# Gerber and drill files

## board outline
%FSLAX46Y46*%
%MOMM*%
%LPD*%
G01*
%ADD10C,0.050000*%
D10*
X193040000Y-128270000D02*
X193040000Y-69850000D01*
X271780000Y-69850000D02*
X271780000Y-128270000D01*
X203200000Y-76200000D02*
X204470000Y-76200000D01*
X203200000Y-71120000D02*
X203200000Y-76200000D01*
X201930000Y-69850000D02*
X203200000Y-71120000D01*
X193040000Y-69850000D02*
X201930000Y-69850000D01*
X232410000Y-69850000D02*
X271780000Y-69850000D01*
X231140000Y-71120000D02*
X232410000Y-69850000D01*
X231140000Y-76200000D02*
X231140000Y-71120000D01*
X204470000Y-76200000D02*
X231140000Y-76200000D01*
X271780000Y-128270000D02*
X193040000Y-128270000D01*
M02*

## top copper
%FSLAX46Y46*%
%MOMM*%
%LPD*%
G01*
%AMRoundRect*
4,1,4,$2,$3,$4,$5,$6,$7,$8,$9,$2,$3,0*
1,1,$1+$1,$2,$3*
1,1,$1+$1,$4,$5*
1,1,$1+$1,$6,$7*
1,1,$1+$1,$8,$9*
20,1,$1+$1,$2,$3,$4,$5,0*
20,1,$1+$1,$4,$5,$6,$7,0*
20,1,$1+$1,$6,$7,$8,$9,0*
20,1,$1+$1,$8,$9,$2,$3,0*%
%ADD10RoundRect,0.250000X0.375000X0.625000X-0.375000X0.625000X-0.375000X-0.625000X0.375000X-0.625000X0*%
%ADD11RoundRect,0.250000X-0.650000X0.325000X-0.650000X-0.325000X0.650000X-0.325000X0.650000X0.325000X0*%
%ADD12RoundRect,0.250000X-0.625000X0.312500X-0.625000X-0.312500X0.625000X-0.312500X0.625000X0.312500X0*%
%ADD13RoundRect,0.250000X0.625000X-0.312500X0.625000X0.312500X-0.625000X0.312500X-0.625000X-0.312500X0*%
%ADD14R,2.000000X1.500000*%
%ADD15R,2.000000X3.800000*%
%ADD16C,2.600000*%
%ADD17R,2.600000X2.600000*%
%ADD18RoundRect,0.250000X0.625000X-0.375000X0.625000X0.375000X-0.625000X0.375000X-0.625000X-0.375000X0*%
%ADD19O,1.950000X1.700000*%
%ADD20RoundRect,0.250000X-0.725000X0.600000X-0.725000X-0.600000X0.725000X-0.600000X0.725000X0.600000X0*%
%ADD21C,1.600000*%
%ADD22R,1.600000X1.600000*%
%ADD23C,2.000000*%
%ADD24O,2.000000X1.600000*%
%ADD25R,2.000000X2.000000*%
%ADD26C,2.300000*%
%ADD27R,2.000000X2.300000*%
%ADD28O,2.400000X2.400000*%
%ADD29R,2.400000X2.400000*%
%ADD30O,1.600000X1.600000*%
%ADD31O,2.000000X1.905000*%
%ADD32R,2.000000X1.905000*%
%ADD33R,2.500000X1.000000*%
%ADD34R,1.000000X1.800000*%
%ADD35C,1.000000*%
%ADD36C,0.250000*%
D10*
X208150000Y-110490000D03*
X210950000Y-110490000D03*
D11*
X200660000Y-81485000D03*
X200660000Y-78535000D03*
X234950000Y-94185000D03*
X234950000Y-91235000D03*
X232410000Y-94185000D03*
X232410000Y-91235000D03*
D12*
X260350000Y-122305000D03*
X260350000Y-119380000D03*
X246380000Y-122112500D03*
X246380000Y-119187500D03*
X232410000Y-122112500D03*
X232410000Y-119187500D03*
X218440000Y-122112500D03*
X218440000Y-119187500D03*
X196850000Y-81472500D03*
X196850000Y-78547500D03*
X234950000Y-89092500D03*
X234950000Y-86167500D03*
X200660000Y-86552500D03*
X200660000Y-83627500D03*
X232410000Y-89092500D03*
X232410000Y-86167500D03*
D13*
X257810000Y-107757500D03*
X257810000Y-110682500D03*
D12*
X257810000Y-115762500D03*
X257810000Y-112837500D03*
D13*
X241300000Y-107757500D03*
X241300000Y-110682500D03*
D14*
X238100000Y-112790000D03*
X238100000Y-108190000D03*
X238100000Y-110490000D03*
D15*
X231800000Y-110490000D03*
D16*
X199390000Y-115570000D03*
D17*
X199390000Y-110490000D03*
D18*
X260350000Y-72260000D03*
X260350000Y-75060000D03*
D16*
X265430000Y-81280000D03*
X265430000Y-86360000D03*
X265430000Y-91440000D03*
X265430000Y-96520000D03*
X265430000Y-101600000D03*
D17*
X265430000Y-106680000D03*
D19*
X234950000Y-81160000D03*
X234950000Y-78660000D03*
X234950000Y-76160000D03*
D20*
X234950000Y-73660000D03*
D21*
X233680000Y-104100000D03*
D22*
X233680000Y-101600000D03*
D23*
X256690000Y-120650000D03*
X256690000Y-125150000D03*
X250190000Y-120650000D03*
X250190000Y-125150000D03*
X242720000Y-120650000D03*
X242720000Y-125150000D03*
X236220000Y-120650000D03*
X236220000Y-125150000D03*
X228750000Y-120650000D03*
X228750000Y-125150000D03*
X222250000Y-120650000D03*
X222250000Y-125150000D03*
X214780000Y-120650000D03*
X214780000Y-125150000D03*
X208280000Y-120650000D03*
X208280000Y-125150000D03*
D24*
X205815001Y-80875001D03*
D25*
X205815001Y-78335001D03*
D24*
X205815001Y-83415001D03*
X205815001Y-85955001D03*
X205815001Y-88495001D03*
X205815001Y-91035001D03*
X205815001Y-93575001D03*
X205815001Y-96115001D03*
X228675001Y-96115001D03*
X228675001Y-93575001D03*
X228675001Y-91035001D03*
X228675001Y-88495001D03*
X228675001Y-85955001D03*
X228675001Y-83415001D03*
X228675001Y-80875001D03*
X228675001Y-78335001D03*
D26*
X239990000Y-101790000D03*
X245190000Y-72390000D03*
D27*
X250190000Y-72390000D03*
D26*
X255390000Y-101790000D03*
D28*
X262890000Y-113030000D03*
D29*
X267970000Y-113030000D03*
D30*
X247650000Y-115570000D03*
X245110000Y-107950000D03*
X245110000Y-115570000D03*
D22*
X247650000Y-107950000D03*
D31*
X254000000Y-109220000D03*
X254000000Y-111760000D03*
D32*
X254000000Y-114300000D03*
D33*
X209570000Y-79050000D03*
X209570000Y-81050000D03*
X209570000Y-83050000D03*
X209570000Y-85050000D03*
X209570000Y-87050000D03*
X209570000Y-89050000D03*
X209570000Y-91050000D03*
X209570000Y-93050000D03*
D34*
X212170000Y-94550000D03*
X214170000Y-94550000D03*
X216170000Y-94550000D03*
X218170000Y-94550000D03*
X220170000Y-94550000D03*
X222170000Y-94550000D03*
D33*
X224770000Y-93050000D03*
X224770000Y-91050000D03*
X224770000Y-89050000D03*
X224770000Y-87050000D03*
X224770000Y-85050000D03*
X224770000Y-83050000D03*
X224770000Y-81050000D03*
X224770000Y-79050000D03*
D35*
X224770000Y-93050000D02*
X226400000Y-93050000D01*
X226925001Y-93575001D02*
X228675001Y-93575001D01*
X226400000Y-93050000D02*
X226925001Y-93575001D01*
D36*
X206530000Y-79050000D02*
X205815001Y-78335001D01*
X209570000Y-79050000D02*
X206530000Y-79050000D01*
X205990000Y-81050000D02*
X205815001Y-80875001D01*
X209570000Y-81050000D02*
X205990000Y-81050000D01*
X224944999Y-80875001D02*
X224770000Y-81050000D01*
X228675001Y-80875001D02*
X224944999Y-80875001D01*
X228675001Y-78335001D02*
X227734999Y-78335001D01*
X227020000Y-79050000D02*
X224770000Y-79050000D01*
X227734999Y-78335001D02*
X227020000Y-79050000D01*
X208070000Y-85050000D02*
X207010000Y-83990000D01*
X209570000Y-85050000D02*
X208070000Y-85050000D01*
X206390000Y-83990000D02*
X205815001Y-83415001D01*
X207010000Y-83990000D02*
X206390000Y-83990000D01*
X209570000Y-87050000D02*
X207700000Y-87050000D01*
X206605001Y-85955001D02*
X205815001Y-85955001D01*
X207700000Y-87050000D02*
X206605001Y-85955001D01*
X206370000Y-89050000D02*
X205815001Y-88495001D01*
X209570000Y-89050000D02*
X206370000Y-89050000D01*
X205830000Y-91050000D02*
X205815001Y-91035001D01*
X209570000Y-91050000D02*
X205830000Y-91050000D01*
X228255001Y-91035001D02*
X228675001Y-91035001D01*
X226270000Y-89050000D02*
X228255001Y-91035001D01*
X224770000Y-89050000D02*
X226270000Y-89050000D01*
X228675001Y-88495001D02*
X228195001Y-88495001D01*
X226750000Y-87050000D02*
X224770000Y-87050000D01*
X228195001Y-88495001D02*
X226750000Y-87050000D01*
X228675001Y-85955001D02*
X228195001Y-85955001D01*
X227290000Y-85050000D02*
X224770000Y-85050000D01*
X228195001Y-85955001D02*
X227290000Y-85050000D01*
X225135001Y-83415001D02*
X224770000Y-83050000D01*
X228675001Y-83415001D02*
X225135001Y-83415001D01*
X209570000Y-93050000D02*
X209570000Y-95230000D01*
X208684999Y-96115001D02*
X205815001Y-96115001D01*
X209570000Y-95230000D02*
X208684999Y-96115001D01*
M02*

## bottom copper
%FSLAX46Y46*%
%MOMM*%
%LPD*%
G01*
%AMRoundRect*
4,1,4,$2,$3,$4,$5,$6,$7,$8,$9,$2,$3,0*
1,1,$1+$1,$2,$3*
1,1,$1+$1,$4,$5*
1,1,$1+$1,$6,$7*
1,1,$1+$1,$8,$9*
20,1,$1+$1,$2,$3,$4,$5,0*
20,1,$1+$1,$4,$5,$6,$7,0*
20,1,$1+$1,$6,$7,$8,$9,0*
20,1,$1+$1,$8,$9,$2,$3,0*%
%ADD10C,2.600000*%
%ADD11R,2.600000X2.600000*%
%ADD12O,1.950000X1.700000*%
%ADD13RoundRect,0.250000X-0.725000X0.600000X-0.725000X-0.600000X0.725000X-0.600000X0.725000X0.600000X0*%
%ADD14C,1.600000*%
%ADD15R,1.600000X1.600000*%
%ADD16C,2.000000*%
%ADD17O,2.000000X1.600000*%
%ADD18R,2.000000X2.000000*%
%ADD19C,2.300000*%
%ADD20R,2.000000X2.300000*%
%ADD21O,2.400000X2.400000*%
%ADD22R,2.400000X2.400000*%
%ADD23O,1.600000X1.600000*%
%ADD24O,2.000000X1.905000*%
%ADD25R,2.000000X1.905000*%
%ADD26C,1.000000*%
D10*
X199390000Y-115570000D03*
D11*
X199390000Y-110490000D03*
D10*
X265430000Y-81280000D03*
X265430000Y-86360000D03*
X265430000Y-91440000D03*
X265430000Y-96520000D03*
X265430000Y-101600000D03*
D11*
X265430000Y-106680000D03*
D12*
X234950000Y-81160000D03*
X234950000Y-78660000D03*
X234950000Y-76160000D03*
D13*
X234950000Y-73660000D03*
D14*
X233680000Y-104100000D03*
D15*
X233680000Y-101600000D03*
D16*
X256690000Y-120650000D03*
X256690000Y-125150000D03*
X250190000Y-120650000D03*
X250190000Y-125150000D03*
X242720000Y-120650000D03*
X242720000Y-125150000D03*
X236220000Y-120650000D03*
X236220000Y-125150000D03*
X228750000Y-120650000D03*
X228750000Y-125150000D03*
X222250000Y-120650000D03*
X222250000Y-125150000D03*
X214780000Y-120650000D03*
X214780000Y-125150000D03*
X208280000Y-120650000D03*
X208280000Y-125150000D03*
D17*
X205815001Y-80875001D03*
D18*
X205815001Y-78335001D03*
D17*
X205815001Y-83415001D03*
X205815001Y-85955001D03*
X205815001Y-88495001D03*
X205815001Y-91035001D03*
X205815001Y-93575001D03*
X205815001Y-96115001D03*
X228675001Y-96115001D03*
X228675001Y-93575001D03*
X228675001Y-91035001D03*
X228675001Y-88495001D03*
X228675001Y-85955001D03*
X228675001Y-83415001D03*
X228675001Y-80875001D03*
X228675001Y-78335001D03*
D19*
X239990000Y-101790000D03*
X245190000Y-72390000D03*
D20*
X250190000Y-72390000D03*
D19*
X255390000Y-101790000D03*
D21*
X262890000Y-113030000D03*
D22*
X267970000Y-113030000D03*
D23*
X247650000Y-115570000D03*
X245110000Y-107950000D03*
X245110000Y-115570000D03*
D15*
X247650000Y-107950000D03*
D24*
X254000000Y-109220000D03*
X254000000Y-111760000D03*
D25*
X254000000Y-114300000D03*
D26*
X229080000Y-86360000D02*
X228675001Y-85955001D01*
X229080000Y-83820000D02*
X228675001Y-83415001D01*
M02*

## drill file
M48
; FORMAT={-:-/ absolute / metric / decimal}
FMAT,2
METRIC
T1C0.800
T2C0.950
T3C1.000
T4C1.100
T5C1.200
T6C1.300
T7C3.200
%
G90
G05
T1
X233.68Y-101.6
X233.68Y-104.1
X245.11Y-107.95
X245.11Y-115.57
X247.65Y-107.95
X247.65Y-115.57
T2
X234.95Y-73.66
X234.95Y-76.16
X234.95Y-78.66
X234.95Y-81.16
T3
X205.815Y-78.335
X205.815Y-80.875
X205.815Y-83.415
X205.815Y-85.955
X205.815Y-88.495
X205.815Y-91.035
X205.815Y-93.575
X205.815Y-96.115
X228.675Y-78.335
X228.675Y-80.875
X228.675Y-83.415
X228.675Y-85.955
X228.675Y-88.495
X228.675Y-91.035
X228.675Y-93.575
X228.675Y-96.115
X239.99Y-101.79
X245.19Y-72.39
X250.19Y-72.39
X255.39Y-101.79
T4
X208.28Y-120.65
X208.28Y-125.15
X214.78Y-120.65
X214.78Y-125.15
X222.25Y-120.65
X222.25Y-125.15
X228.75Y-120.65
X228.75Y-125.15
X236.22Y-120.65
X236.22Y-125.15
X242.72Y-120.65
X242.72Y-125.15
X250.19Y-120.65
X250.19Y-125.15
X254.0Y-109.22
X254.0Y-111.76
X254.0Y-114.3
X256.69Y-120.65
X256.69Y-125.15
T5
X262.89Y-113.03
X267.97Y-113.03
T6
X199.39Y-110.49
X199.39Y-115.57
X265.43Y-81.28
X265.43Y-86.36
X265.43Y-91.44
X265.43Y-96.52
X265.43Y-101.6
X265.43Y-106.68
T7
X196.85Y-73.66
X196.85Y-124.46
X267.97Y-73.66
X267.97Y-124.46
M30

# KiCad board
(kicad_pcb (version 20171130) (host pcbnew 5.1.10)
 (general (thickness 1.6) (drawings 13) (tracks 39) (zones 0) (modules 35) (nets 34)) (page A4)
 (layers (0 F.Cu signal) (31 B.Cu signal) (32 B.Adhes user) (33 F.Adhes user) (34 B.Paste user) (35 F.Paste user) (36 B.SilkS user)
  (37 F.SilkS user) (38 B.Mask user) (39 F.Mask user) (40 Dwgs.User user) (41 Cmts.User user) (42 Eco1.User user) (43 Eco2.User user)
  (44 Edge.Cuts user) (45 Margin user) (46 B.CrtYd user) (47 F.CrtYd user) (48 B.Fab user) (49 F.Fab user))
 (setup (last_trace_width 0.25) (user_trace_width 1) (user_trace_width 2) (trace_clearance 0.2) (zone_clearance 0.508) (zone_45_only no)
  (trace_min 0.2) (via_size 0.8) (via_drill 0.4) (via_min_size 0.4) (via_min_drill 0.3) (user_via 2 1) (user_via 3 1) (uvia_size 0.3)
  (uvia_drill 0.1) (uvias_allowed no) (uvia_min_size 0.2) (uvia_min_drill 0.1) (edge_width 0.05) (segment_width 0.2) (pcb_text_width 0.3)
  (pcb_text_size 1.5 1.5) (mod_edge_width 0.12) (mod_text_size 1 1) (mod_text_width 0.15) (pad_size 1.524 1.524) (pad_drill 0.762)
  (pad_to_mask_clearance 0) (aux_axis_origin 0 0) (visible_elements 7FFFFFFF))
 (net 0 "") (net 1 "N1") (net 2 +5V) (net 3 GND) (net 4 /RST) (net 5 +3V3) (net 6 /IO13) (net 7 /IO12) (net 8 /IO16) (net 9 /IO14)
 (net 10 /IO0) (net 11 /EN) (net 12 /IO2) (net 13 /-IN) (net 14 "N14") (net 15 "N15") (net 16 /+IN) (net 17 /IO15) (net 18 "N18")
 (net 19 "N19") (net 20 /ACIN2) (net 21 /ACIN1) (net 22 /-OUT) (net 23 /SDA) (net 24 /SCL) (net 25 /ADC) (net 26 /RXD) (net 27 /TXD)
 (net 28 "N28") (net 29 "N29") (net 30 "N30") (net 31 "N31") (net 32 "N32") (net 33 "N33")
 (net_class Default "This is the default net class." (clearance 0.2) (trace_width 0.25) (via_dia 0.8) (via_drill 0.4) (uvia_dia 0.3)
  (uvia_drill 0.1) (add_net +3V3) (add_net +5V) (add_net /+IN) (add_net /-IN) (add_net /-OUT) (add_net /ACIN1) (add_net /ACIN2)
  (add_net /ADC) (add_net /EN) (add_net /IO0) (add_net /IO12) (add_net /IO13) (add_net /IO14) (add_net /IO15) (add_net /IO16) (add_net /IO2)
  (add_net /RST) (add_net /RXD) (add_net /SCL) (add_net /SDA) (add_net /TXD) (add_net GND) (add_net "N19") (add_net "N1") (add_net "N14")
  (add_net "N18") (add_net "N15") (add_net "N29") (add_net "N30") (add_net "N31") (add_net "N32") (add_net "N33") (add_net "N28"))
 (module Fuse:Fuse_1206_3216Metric (layer F.Cu) (at 209.55 110.49 180)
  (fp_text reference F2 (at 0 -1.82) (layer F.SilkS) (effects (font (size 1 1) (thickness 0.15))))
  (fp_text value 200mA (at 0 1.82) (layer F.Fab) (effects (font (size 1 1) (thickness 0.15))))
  (pad 2 smd roundrect (at 1.4 0 180) (size 1.25 1.75) (layers F.Cu F.Paste F.Mask) (roundrect_rratio 0.2) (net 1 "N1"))
  (pad 1 smd roundrect (at -1.4 0 180) (size 1.25 1.75) (layers F.Cu F.Paste F.Mask) (roundrect_rratio 0.2) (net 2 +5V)))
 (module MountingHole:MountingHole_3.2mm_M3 (layer F.Cu) (at 267.97 124.46)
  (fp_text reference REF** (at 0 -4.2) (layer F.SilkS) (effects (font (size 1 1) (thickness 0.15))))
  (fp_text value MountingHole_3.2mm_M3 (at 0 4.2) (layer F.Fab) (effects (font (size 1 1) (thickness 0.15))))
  (pad 1 np_thru_hole circle (at 0 0) (size 3.2 3.2) (drill 3.2) (layers *.Cu *.Mask)))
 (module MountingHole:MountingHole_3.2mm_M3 (layer F.Cu) (at 196.85 124.46)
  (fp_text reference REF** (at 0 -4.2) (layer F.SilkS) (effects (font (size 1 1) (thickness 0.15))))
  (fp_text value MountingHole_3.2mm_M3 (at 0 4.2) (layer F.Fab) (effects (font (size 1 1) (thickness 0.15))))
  (pad 1 np_thru_hole circle (at 0 0) (size 3.2 3.2) (drill 3.2) (layers *.Cu *.Mask)))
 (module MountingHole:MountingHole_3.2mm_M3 (layer F.Cu) (at 196.85 73.66)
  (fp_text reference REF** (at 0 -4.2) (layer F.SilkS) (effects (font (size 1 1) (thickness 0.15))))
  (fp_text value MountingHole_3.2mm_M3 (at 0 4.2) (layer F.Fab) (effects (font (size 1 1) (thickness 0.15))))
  (pad 1 np_thru_hole circle (at 0 0) (size 3.2 3.2) (drill 3.2) (layers *.Cu *.Mask)))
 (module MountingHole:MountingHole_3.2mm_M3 (layer F.Cu) (at 267.97 73.66)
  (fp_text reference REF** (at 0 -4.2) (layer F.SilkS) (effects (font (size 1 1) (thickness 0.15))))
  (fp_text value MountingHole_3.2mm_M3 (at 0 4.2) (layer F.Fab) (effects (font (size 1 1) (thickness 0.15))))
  (pad 1 np_thru_hole circle (at 0 0) (size 3.2 3.2) (drill 3.2) (layers *.Cu *.Mask)))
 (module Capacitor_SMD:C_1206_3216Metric (layer F.Cu) (at 200.66 80.01 270)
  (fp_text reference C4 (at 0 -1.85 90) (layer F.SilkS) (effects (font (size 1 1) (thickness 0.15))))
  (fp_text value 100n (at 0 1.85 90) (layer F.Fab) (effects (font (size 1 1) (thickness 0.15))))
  (pad 2 smd roundrect (at 1.475 0 270) (size 1.15 1.8) (layers F.Cu F.Paste F.Mask) (roundrect_rratio 0.217391) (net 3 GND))
  (pad 1 smd roundrect (at -1.475 0 270) (size 1.15 1.8) (layers F.Cu F.Paste F.Mask) (roundrect_rratio 0.217391) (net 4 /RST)))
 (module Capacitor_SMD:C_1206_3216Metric (layer F.Cu) (at 234.95 92.71 270)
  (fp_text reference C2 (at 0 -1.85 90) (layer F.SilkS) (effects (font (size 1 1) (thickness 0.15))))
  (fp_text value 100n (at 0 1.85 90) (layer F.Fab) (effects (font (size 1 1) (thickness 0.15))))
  (pad 2 smd roundrect (at 1.475 0 270) (size 1.15 1.8) (layers F.Cu F.Paste F.Mask) (roundrect_rratio 0.217391) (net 3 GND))
  (pad 1 smd roundrect (at -1.475 0 270) (size 1.15 1.8) (layers F.Cu F.Paste F.Mask) (roundrect_rratio 0.217391) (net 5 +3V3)))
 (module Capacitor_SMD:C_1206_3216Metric (layer F.Cu) (at 232.41 92.71 270)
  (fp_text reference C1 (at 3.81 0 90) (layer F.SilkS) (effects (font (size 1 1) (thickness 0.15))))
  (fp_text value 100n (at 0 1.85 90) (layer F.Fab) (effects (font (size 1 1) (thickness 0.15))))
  (pad 2 smd roundrect (at 1.475 0 270) (size 1.15 1.8) (layers F.Cu F.Paste F.Mask) (roundrect_rratio 0.217391) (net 3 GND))
  (pad 1 smd roundrect (at -1.475 0 270) (size 1.15 1.8) (layers F.Cu F.Paste F.Mask) (roundrect_rratio 0.217391) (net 2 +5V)))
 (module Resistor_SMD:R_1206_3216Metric (layer F.Cu) (at 260.35 120.8425 270)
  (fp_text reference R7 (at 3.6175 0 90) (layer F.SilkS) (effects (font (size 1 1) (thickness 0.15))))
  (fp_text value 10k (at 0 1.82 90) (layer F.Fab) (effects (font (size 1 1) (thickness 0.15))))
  (pad 2 smd roundrect (at 1.4625 0 270) (size 1.125 1.75) (layers F.Cu F.Paste F.Mask) (roundrect_rratio 0.222222) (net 3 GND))
  (pad 1 smd roundrect (at -1.4625 0 270) (size 1.125 1.75) (layers F.Cu F.Paste F.Mask) (roundrect_rratio 0.222222) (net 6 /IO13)))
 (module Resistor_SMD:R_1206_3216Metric (layer F.Cu) (at 246.38 120.65 270)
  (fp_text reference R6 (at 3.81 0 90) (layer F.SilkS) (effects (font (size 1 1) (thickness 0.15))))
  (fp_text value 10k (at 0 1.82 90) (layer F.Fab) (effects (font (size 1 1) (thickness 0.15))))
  (pad 2 smd roundrect (at 1.4625 0 270) (size 1.125 1.75) (layers F.Cu F.Paste F.Mask) (roundrect_rratio 0.222222) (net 3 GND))
  (pad 1 smd roundrect (at -1.4625 0 270) (size 1.125 1.75) (layers F.Cu F.Paste F.Mask) (roundrect_rratio 0.222222) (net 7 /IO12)))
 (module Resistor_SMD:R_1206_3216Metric (layer F.Cu) (at 232.41 120.65 270)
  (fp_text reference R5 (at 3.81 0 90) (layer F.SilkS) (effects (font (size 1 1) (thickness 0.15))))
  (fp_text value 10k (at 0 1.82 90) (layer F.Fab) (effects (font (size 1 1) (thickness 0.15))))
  (pad 2 smd roundrect (at 1.4625 0 270) (size 1.125 1.75) (layers F.Cu F.Paste F.Mask) (roundrect_rratio 0.222222) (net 3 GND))
  (pad 1 smd roundrect (at -1.4625 0 270) (size 1.125 1.75) (layers F.Cu F.Paste F.Mask) (roundrect_rratio 0.222222) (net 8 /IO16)))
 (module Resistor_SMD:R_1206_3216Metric (layer F.Cu) (at 218.44 120.65 270)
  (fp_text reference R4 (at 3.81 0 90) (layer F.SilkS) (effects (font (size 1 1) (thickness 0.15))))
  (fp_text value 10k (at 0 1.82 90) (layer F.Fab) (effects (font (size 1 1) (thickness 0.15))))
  (pad 2 smd roundrect (at 1.4625 0 270) (size 1.125 1.75) (layers F.Cu F.Paste F.Mask) (roundrect_rratio 0.222222) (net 3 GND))
  (pad 1 smd roundrect (at -1.4625 0 270) (size 1.125 1.75) (layers F.Cu F.Paste F.Mask) (roundrect_rratio 0.222222) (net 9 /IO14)))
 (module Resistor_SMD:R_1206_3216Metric (layer F.Cu) (at 196.85 80.01 270)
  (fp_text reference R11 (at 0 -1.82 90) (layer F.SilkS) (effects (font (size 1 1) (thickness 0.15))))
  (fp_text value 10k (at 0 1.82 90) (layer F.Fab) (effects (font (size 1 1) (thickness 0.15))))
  (pad 2 smd roundrect (at 1.4625 0 270) (size 1.125 1.75) (layers F.Cu F.Paste F.Mask) (roundrect_rratio 0.222222) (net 5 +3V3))
  (pad 1 smd roundrect (at -1.4625 0 270) (size 1.125 1.75) (layers F.Cu F.Paste F.Mask) (roundrect_rratio 0.222222) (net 4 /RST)))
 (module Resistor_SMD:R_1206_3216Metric (layer F.Cu) (at 234.95 87.63 270)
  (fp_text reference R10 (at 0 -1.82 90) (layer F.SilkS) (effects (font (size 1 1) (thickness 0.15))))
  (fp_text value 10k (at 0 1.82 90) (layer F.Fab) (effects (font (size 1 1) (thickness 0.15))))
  (pad 2 smd roundrect (at 1.4625 0 270) (size 1.125 1.75) (layers F.Cu F.Paste F.Mask) (roundrect_rratio 0.222222) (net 5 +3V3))
  (pad 1 smd roundrect (at -1.4625 0 270) (size 1.125 1.75) (layers F.Cu F.Paste F.Mask) (roundrect_rratio 0.222222) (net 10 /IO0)))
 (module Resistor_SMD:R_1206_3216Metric (layer F.Cu) (at 200.66 85.09 270)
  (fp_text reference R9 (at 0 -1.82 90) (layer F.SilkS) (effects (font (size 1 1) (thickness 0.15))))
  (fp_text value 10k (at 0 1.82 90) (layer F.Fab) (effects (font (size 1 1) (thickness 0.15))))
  (pad 2 smd roundrect (at 1.4625 0 270) (size 1.125 1.75) (layers F.Cu F.Paste F.Mask) (roundrect_rratio 0.222222) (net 5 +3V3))
  (pad 1 smd roundrect (at -1.4625 0 270) (size 1.125 1.75) (layers F.Cu F.Paste F.Mask) (roundrect_rratio 0.222222) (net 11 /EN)))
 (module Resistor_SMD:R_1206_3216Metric (layer F.Cu) (at 232.41 87.63 270)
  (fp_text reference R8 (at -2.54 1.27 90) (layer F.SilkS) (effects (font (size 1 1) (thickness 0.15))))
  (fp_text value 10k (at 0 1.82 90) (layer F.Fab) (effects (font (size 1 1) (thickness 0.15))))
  (pad 2 smd roundrect (at 1.4625 0 270) (size 1.125 1.75) (layers F.Cu F.Paste F.Mask) (roundrect_rratio 0.222222) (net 5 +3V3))
  (pad 1 smd roundrect (at -1.4625 0 270) (size 1.125 1.75) (layers F.Cu F.Paste F.Mask) (roundrect_rratio 0.222222) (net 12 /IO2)))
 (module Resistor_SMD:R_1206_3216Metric (layer F.Cu) (at 257.81 109.22 90)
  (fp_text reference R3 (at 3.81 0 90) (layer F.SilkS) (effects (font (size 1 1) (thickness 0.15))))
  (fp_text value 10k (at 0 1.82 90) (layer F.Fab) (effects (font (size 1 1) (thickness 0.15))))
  (pad 2 smd roundrect (at 1.4625 0 90) (size 1.125 1.75) (layers F.Cu F.Paste F.Mask) (roundrect_rratio 0.222222) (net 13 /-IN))
  (pad 1 smd roundrect (at -1.4625 0 90) (size 1.125 1.75) (layers F.Cu F.Paste F.Mask) (roundrect_rratio 0.222222) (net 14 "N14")))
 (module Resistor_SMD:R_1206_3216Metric (layer F.Cu) (at 257.81 114.3 270)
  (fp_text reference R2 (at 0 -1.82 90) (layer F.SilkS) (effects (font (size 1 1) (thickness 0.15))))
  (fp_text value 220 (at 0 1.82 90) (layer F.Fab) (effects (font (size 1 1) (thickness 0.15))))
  (pad 2 smd roundrect (at 1.4625 0 270) (size 1.125 1.75) (layers F.Cu F.Paste F.Mask) (roundrect_rratio 0.222222) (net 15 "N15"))
  (pad 1 smd roundrect (at -1.4625 0 270) (size 1.125 1.75) (layers F.Cu F.Paste F.Mask) (roundrect_rratio 0.222222) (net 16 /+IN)))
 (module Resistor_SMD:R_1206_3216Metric (layer F.Cu) (at 241.3 109.22 90)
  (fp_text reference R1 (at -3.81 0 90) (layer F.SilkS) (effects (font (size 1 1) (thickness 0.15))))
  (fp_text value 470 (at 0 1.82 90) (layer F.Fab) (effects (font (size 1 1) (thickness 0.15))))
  (pad 2 smd roundrect (at 1.4625 0 90) (size 1.125 1.75) (layers F.Cu F.Paste F.Mask) (roundrect_rratio 0.222222) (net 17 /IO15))
  (pad 1 smd roundrect (at -1.4625 0 90) (size 1.125 1.75) (layers F.Cu F.Paste F.Mask) (roundrect_rratio 0.222222) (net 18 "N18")))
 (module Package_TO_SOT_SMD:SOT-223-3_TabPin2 (layer F.Cu) (at 234.95 110.49 180)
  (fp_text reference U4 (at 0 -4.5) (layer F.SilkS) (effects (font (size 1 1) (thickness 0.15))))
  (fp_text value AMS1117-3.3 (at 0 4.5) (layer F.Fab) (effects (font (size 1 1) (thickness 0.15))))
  (pad 1 smd rect (at -3.15 -2.3 180) (size 2 1.5) (layers F.Cu F.Paste F.Mask) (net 3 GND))
  (pad 3 smd rect (at -3.15 2.3 180) (size 2 1.5) (layers F.Cu F.Paste F.Mask) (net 2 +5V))
  (pad 2 smd rect (at -3.15 0 180) (size 2 1.5) (layers F.Cu F.Paste F.Mask) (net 5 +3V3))
  (pad 2 smd rect (at 3.15 0 180) (size 2 3.8) (layers F.Cu F.Paste F.Mask) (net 5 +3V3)))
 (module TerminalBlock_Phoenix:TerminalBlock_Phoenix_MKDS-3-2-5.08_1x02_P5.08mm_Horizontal (layer F.Cu) (at 199.39 110.49 270)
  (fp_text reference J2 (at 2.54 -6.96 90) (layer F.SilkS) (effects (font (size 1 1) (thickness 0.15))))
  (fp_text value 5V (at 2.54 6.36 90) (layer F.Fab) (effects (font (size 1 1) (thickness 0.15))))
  (pad 2 thru_hole circle (at 5.08 0 270) (size 2.6 2.6) (drill 1.3) (layers *.Cu *.Mask) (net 3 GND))
  (pad 1 thru_hole rect (at 0 0 270) (size 2.6 2.6) (drill 1.3) (layers *.Cu *.Mask) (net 1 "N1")))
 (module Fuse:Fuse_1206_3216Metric (layer F.Cu) (at 260.35 73.66 90)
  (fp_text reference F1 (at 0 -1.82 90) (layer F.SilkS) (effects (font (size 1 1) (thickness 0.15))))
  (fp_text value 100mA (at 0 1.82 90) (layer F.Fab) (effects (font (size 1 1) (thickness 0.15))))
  (pad 2 smd roundrect (at 1.4 0 90) (size 1.25 1.75) (layers F.Cu F.Paste F.Mask) (roundrect_rratio 0.2) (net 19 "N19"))
  (pad 1 smd roundrect (at -1.4 0 90) (size 1.25 1.75) (layers F.Cu F.Paste F.Mask) (roundrect_rratio 0.2) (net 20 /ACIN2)))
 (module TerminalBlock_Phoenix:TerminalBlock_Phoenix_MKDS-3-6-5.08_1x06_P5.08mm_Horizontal (layer F.Cu) (at 265.43 106.68 90)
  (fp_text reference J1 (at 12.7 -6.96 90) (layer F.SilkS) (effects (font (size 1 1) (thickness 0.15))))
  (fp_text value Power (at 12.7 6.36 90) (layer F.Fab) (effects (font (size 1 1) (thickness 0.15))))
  (pad 6 thru_hole circle (at 25.4 0 90) (size 2.6 2.6) (drill 1.3) (layers *.Cu *.Mask) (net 20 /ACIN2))
  (pad 5 thru_hole circle (at 20.32 0 90) (size 2.6 2.6) (drill 1.3) (layers *.Cu *.Mask) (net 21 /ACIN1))
  (pad 4 thru_hole circle (at 15.24 0 90) (size 2.6 2.6) (drill 1.3) (layers *.Cu *.Mask) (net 13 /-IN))
  (pad 3 thru_hole circle (at 10.16 0 90) (size 2.6 2.6) (drill 1.3) (layers *.Cu *.Mask) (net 16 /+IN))
  (pad 2 thru_hole circle (at 5.08 0 90) (size 2.6 2.6) (drill 1.3) (layers *.Cu *.Mask) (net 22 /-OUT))
  (pad 1 thru_hole rect (at 0 0 90) (size 2.6 2.6) (drill 1.3) (layers *.Cu *.Mask) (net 16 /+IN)))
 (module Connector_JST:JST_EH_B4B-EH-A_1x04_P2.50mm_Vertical (layer F.Cu) (at 234.95 73.66 270)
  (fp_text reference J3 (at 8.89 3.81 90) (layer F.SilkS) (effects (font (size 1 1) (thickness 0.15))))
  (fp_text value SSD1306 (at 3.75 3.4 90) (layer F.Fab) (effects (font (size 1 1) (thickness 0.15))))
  (pad 4 thru_hole oval (at 7.5 0 270) (size 1.7 1.95) (drill 0.95) (layers *.Cu *.Mask) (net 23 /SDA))
  (pad 3 thru_hole oval (at 5 0 270) (size 1.7 1.95) (drill 0.95) (layers *.Cu *.Mask) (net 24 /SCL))
  (pad 2 thru_hole oval (at 2.5 0 270) (size 1.7 1.95) (drill 0.95) (layers *.Cu *.Mask) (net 2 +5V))
  (pad 1 thru_hole roundrect (at 0 0 270) (size 1.7 1.95) (drill 0.95) (layers *.Cu *.Mask) (roundrect_rratio 0.147059) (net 3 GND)))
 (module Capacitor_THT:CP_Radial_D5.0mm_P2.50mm (layer F.Cu) (at 233.68 101.6 270)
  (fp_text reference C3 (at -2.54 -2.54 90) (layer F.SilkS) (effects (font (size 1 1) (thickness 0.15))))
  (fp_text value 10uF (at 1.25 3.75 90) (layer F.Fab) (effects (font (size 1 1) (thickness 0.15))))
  (pad 2 thru_hole circle (at 2.5 0 270) (size 1.6 1.6) (drill 0.8) (layers *.Cu *.Mask) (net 3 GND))
  (pad 1 thru_hole rect (at 0 0 270) (size 1.6 1.6) (drill 0.8) (layers *.Cu *.Mask) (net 5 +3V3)))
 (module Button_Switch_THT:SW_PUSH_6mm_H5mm (layer F.Cu) (at 250.19 120.65)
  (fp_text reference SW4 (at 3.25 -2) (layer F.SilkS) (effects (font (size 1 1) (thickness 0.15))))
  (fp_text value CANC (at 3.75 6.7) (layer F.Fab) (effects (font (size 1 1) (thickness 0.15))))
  (pad 1 thru_hole circle (at 6.5 0 90) (size 2 2) (drill 1.1) (layers *.Cu *.Mask) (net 6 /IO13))
  (pad 2 thru_hole circle (at 6.5 4.5 90) (size 2 2) (drill 1.1) (layers *.Cu *.Mask) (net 5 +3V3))
  (pad 1 thru_hole circle (at 0 0 90) (size 2 2) (drill 1.1) (layers *.Cu *.Mask) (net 6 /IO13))
  (pad 2 thru_hole circle (at 0 4.5 90) (size 2 2) (drill 1.1) (layers *.Cu *.Mask) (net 5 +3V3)))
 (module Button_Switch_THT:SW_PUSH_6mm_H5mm (layer F.Cu) (at 236.22 120.65)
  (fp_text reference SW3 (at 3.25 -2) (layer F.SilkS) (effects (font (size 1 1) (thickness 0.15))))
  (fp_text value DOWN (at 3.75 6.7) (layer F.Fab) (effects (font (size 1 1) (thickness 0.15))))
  (pad 1 thru_hole circle (at 6.5 0 90) (size 2 2) (drill 1.1) (layers *.Cu *.Mask) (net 7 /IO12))
  (pad 2 thru_hole circle (at 6.5 4.5 90) (size 2 2) (drill 1.1) (layers *.Cu *.Mask) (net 5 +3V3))
  (pad 1 thru_hole circle (at 0 0 90) (size 2 2) (drill 1.1) (layers *.Cu *.Mask) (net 7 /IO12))
  (pad 2 thru_hole circle (at 0 4.5 90) (size 2 2) (drill 1.1) (layers *.Cu *.Mask) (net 5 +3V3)))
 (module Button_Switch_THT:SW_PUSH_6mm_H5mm (layer F.Cu) (at 222.25 120.65)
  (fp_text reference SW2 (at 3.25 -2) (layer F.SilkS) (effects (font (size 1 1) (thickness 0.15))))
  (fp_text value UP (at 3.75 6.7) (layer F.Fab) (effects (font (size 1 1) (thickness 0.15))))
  (pad 1 thru_hole circle (at 6.5 0 90) (size 2 2) (drill 1.1) (layers *.Cu *.Mask) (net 8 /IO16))
  (pad 2 thru_hole circle (at 6.5 4.5 90) (size 2 2) (drill 1.1) (layers *.Cu *.Mask) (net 5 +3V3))
  (pad 1 thru_hole circle (at 0 0 90) (size 2 2) (drill 1.1) (layers *.Cu *.Mask) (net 8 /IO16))
  (pad 2 thru_hole circle (at 0 4.5 90) (size 2 2) (drill 1.1) (layers *.Cu *.Mask) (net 5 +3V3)))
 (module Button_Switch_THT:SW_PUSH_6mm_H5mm (layer F.Cu) (at 208.28 120.65)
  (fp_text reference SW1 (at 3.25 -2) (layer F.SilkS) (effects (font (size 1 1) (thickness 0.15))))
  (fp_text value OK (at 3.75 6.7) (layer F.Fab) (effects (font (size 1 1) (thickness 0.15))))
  (pad 1 thru_hole circle (at 6.5 0 90) (size 2 2) (drill 1.1) (layers *.Cu *.Mask) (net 9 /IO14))
  (pad 2 thru_hole circle (at 6.5 4.5 90) (size 2 2) (drill 1.1) (layers *.Cu *.Mask) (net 5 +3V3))
  (pad 1 thru_hole circle (at 0 0 90) (size 2 2) (drill 1.1) (layers *.Cu *.Mask) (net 9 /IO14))
  (pad 2 thru_hole circle (at 0 4.5 90) (size 2 2) (drill 1.1) (layers *.Cu *.Mask) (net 5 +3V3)))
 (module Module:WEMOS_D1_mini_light (layer F.Cu) (at 205.815001 78.335001)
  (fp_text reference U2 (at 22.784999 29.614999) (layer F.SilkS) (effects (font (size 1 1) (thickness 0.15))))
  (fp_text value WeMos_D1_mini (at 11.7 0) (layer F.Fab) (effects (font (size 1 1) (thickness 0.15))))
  (pad 2 thru_hole oval (at 0 2.54) (size 2 1.6) (drill 1) (layers *.Cu *.Mask) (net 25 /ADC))
  (pad 1 thru_hole rect (at 0 0) (size 2 2) (drill 1) (layers *.Cu *.Mask) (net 4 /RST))
  (pad 3 thru_hole oval (at 0 5.08) (size 2 1.6) (drill 1) (layers *.Cu *.Mask) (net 8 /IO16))
  (pad 4 thru_hole oval (at 0 7.62) (size 2 1.6) (drill 1) (layers *.Cu *.Mask) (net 9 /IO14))
  (pad 5 thru_hole oval (at 0 10.16) (size 2 1.6) (drill 1) (layers *.Cu *.Mask) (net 7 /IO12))
  (pad 6 thru_hole oval (at 0 12.7) (size 2 1.6) (drill 1) (layers *.Cu *.Mask) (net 6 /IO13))
  (pad 7 thru_hole oval (at 0 15.24) (size 2 1.6) (drill 1) (layers *.Cu *.Mask) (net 17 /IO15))
  (pad 8 thru_hole oval (at 0 17.78) (size 2 1.6) (drill 1) (layers *.Cu *.Mask) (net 5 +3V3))
  (pad 9 thru_hole oval (at 22.86 17.78) (size 2 1.6) (drill 1) (layers *.Cu *.Mask) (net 2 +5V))
  (pad 10 thru_hole oval (at 22.86 15.24) (size 2 1.6) (drill 1) (layers *.Cu *.Mask) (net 3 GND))
  (pad 11 thru_hole oval (at 22.86 12.7) (size 2 1.6) (drill 1) (layers *.Cu *.Mask) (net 12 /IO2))
  (pad 12 thru_hole oval (at 22.86 10.16) (size 2 1.6) (drill 1) (layers *.Cu *.Mask) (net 10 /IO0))
  (pad 13 thru_hole oval (at 22.86 7.62) (size 2 1.6) (drill 1) (layers *.Cu *.Mask) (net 23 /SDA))
  (pad 14 thru_hole oval (at 22.86 5.08) (size 2 1.6) (drill 1) (layers *.Cu *.Mask) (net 24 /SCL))
  (pad 15 thru_hole oval (at 22.86 2.54) (size 2 1.6) (drill 1) (layers *.Cu *.Mask) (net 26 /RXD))
  (pad 16 thru_hole oval (at 22.86 0) (size 2 1.6) (drill 1) (layers *.Cu *.Mask) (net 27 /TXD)))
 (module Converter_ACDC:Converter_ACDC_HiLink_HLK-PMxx (layer F.Cu) (at 250.19 72.39 270)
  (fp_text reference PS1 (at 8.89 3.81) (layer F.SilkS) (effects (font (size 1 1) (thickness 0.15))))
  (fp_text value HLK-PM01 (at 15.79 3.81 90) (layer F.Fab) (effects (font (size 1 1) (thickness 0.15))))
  (pad 4 thru_hole circle (at 29.4 10.2 270) (size 2.3 2.3) (drill 1) (layers *.Cu *.Mask) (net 2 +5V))
  (pad 2 thru_hole circle (at 0 5 270) (size 2.3 2.3) (drill 1) (layers *.Cu *.Mask) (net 21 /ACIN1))
  (pad 1 thru_hole rect (at 0 0 270) (size 2.3 2) (drill 1) (layers *.Cu *.Mask) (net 19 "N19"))
  (pad 3 thru_hole circle (at 29.4 -5.2 270) (size 2.3 2.3) (drill 1) (layers *.Cu *.Mask) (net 3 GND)))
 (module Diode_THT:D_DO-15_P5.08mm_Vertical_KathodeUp (layer F.Cu) (at 267.97 113.03 180)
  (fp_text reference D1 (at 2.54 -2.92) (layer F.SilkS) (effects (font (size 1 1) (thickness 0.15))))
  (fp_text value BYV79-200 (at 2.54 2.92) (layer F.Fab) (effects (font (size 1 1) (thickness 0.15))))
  (pad 2 thru_hole oval (at 5.08 0 180) (size 2.4 2.4) (drill 1.2) (layers *.Cu *.Mask) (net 22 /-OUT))
  (pad 1 thru_hole rect (at 0 0 180) (size 2.4 2.4) (drill 1.2) (layers *.Cu *.Mask) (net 16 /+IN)))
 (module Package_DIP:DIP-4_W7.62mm (layer F.Cu) (at 247.65 107.95 270)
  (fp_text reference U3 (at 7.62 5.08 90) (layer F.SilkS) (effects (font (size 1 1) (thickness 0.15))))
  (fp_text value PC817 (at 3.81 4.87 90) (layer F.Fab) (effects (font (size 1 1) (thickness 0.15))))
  (pad 4 thru_hole oval (at 7.62 0 270) (size 1.6 1.6) (drill 0.8) (layers *.Cu *.Mask) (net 15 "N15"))
  (pad 2 thru_hole oval (at 0 2.54 270) (size 1.6 1.6) (drill 0.8) (layers *.Cu *.Mask) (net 3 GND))
  (pad 3 thru_hole oval (at 7.62 2.54 270) (size 1.6 1.6) (drill 0.8) (layers *.Cu *.Mask) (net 14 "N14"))
  (pad 1 thru_hole rect (at 0 0 270) (size 1.6 1.6) (drill 0.8) (layers *.Cu *.Mask) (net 18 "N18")))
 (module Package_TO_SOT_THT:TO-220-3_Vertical (layer F.Cu) (at 254 114.3 90)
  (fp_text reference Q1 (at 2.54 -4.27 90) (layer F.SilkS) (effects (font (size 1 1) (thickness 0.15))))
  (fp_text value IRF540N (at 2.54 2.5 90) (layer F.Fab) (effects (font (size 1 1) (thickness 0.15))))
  (pad 3 thru_hole oval (at 5.08 0 90) (size 1.905 2) (drill 1.1) (layers *.Cu *.Mask) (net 13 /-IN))
  (pad 2 thru_hole oval (at 2.54 0 90) (size 1.905 2) (drill 1.1) (layers *.Cu *.Mask) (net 22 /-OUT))
  (pad 1 thru_hole rect (at 0 0 90) (size 1.905 2) (drill 1.1) (layers *.Cu *.Mask) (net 14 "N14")))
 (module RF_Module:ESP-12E (layer F.Cu) (at 217.17 82.55)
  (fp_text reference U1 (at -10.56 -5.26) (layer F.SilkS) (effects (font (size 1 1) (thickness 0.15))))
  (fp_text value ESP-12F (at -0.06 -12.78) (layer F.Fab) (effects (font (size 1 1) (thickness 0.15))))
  (pad 1 smd rect (at -7.6 -3.5) (size 2.5 1) (layers F.Cu F.Paste F.Mask) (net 4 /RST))
  (pad 2 smd rect (at -7.6 -1.5) (size 2.5 1) (layers F.Cu F.Paste F.Mask) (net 25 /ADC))
  (pad 3 smd rect (at -7.6 0.5) (size 2.5 1) (layers F.Cu F.Paste F.Mask) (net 11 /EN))
  (pad 4 smd rect (at -7.6 2.5) (size 2.5 1) (layers F.Cu F.Paste F.Mask) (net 8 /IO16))
  (pad 5 smd rect (at -7.6 4.5) (size 2.5 1) (layers F.Cu F.Paste F.Mask) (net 9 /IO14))
  (pad 6 smd rect (at -7.6 6.5) (size 2.5 1) (layers F.Cu F.Paste F.Mask) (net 7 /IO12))
  (pad 7 smd rect (at -7.6 8.5) (size 2.5 1) (layers F.Cu F.Paste F.Mask) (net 6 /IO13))
  (pad 8 smd rect (at -7.6 10.5) (size 2.5 1) (layers F.Cu F.Paste F.Mask) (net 5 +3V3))
  (pad 9 smd rect (at -5 12) (size 1 1.8) (layers F.Cu F.Paste F.Mask) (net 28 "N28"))
  (pad 10 smd rect (at -3 12) (size 1 1.8) (layers F.Cu F.Paste F.Mask) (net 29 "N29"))
  (pad 11 smd rect (at -1 12) (size 1 1.8) (layers F.Cu F.Paste F.Mask) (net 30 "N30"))
  (pad 12 smd rect (at 1 12) (size 1 1.8) (layers F.Cu F.Paste F.Mask) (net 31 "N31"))
  (pad 13 smd rect (at 3 12) (size 1 1.8) (layers F.Cu F.Paste F.Mask) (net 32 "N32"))
  (pad 14 smd rect (at 5 12) (size 1 1.8) (layers F.Cu F.Paste F.Mask) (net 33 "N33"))
  (pad 15 smd rect (at 7.6 10.5) (size 2.5 1) (layers F.Cu F.Paste F.Mask) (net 3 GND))
  (pad 16 smd rect (at 7.6 8.5) (size 2.5 1) (layers F.Cu F.Paste F.Mask) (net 17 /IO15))
  (pad 17 smd rect (at 7.6 6.5) (size 2.5 1) (layers F.Cu F.Paste F.Mask) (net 12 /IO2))
  (pad 18 smd rect (at 7.6 4.5) (size 2.5 1) (layers F.Cu F.Paste F.Mask) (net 10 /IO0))
  (pad 19 smd rect (at 7.6 2.5) (size 2.5 1) (layers F.Cu F.Paste F.Mask) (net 23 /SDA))
  (pad 20 smd rect (at 7.6 0.5) (size 2.5 1) (layers F.Cu F.Paste F.Mask) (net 24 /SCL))
  (pad 21 smd rect (at 7.6 -1.5) (size 2.5 1) (layers F.Cu F.Paste F.Mask) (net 26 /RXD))
  (pad 22 smd rect (at 7.6 -3.5) (size 2.5 1) (layers F.Cu F.Paste F.Mask) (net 27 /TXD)))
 (gr_line (start 193.04 128.27) (end 193.04 69.85) (layer Edge.Cuts) (width 0.05))
 (gr_line (start 271.78 69.85) (end 271.78 128.27) (layer Edge.Cuts) (width 0.05))
 (gr_line (start 203.2 76.2) (end 204.47 76.2) (layer Edge.Cuts) (width 0.05))
 (gr_line (start 203.2 71.12) (end 203.2 76.2) (layer Edge.Cuts) (width 0.05))
 (gr_line (start 201.93 69.85) (end 203.2 71.12) (layer Edge.Cuts) (width 0.05))
 (gr_line (start 193.04 69.85) (end 201.93 69.85) (layer Edge.Cuts) (width 0.05))
 (gr_line (start 232.41 69.85) (end 271.78 69.85) (layer Edge.Cuts) (width 0.05))
 (gr_line (start 231.14 71.12) (end 232.41 69.85) (layer Edge.Cuts) (width 0.05))
 (gr_line (start 231.14 76.2) (end 231.14 71.12) (layer Edge.Cuts) (width 0.05))
 (gr_line (start 204.47 76.2) (end 231.14 76.2) (layer Edge.Cuts) (width 0.05))
 (gr_line (start 271.78 128.27) (end 193.04 128.27) (layer Edge.Cuts) (width 0.05))
 (segment (start 224.77 93.05) (end 226.4 93.05) (width 1) (layer F.Cu) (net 3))
 (segment (start 226.925001 93.575001) (end 228.675001 93.575001) (width 1) (layer F.Cu) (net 3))
 (segment (start 226.4 93.05) (end 226.925001 93.575001) (width 1) (layer F.Cu) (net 3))
 (segment (start 206.53 79.05) (end 205.815001 78.335001) (width 0.25) (layer F.Cu) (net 4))
 (segment (start 209.57 79.05) (end 206.53 79.05) (width 0.25) (layer F.Cu) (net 4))
 (segment (start 205.99 81.05) (end 205.815001 80.875001) (width 0.25) (layer F.Cu) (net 25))
 (segment (start 209.57 81.05) (end 205.99 81.05) (width 0.25) (layer F.Cu) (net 25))
 (segment (start 224.944999 80.875001) (end 224.77 81.05) (width 0.25) (layer F.Cu) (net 26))
 (segment (start 228.675001 80.875001) (end 224.944999 80.875001) (width 0.25) (layer F.Cu) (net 26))
 (segment (start 228.675001 78.335001) (end 227.734999 78.335001) (width 0.25) (layer F.Cu) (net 27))
 (segment (start 227.02 79.05) (end 224.77 79.05) (width 0.25) (layer F.Cu) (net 27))
 (segment (start 227.734999 78.335001) (end 227.02 79.05) (width 0.25) (layer F.Cu) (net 27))
 (segment (start 208.07 85.05) (end 207.01 83.99) (width 0.25) (layer F.Cu) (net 8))
 (segment (start 209.57 85.05) (end 208.07 85.05) (width 0.25) (layer F.Cu) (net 8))
 (segment (start 206.39 83.99) (end 205.815001 83.415001) (width 0.25) (layer F.Cu) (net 8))
 (segment (start 207.01 83.99) (end 206.39 83.99) (width 0.25) (layer F.Cu) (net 8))
 (segment (start 209.57 87.05) (end 207.7 87.05) (width 0.25) (layer F.Cu) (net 9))
 (segment (start 206.605001 85.955001) (end 205.815001 85.955001) (width 0.25) (layer F.Cu) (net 9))
 (segment (start 207.7 87.05) (end 206.605001 85.955001) (width 0.25) (layer F.Cu) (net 9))
 (segment (start 206.37 89.05) (end 205.815001 88.495001) (width 0.25) (layer F.Cu) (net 7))
 (segment (start 209.57 89.05) (end 206.37 89.05) (width 0.25) (layer F.Cu) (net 7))
 (segment (start 205.83 91.05) (end 205.815001 91.035001) (width 0.25) (layer F.Cu) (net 6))
 (segment (start 209.57 91.05) (end 205.83 91.05) (width 0.25) (layer F.Cu) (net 6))
 (segment (start 228.255001 91.035001) (end 228.675001 91.035001) (width 0.25) (layer F.Cu) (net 12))
 (segment (start 226.27 89.05) (end 228.255001 91.035001) (width 0.25) (layer F.Cu) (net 12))
 (segment (start 224.77 89.05) (end 226.27 89.05) (width 0.25) (layer F.Cu) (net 12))
 (segment (start 228.675001 88.495001) (end 228.195001 88.495001) (width 0.25) (layer F.Cu) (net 10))
 (segment (start 226.75 87.05) (end 224.77 87.05) (width 0.25) (layer F.Cu) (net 10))
 (segment (start 228.195001 88.495001) (end 226.75 87.05) (width 0.25) (layer F.Cu) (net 10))
 (segment (start 228.675001 85.955001) (end 228.195001 85.955001) (width 0.25) (layer F.Cu) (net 23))
 (segment (start 227.29 85.05) (end 224.77 85.05) (width 0.25) (layer F.Cu) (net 23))
 (segment (start 228.195001 85.955001) (end 227.29 85.05) (width 0.25) (layer F.Cu) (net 23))
 (segment (start 229.08 86.36) (end 228.675001 85.955001) (width 1) (layer B.Cu) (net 23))
 (segment (start 225.135001 83.415001) (end 224.77 83.05) (width 0.25) (layer F.Cu) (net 24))
 (segment (start 228.675001 83.415001) (end 225.135001 83.415001) (width 0.25) (layer F.Cu) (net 24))
 (segment (start 229.08 83.82) (end 228.675001 83.415001) (width 1) (layer B.Cu) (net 24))
 (segment (start 209.57 93.05) (end 209.57 95.23) (width 0.25) (layer F.Cu) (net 5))
 (segment (start 208.684999 96.115001) (end 205.815001 96.115001) (width 0.25) (layer F.Cu) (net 5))
 (segment (start 209.57 95.23) (end 208.684999 96.115001) (width 0.25) (layer F.Cu) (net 5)))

